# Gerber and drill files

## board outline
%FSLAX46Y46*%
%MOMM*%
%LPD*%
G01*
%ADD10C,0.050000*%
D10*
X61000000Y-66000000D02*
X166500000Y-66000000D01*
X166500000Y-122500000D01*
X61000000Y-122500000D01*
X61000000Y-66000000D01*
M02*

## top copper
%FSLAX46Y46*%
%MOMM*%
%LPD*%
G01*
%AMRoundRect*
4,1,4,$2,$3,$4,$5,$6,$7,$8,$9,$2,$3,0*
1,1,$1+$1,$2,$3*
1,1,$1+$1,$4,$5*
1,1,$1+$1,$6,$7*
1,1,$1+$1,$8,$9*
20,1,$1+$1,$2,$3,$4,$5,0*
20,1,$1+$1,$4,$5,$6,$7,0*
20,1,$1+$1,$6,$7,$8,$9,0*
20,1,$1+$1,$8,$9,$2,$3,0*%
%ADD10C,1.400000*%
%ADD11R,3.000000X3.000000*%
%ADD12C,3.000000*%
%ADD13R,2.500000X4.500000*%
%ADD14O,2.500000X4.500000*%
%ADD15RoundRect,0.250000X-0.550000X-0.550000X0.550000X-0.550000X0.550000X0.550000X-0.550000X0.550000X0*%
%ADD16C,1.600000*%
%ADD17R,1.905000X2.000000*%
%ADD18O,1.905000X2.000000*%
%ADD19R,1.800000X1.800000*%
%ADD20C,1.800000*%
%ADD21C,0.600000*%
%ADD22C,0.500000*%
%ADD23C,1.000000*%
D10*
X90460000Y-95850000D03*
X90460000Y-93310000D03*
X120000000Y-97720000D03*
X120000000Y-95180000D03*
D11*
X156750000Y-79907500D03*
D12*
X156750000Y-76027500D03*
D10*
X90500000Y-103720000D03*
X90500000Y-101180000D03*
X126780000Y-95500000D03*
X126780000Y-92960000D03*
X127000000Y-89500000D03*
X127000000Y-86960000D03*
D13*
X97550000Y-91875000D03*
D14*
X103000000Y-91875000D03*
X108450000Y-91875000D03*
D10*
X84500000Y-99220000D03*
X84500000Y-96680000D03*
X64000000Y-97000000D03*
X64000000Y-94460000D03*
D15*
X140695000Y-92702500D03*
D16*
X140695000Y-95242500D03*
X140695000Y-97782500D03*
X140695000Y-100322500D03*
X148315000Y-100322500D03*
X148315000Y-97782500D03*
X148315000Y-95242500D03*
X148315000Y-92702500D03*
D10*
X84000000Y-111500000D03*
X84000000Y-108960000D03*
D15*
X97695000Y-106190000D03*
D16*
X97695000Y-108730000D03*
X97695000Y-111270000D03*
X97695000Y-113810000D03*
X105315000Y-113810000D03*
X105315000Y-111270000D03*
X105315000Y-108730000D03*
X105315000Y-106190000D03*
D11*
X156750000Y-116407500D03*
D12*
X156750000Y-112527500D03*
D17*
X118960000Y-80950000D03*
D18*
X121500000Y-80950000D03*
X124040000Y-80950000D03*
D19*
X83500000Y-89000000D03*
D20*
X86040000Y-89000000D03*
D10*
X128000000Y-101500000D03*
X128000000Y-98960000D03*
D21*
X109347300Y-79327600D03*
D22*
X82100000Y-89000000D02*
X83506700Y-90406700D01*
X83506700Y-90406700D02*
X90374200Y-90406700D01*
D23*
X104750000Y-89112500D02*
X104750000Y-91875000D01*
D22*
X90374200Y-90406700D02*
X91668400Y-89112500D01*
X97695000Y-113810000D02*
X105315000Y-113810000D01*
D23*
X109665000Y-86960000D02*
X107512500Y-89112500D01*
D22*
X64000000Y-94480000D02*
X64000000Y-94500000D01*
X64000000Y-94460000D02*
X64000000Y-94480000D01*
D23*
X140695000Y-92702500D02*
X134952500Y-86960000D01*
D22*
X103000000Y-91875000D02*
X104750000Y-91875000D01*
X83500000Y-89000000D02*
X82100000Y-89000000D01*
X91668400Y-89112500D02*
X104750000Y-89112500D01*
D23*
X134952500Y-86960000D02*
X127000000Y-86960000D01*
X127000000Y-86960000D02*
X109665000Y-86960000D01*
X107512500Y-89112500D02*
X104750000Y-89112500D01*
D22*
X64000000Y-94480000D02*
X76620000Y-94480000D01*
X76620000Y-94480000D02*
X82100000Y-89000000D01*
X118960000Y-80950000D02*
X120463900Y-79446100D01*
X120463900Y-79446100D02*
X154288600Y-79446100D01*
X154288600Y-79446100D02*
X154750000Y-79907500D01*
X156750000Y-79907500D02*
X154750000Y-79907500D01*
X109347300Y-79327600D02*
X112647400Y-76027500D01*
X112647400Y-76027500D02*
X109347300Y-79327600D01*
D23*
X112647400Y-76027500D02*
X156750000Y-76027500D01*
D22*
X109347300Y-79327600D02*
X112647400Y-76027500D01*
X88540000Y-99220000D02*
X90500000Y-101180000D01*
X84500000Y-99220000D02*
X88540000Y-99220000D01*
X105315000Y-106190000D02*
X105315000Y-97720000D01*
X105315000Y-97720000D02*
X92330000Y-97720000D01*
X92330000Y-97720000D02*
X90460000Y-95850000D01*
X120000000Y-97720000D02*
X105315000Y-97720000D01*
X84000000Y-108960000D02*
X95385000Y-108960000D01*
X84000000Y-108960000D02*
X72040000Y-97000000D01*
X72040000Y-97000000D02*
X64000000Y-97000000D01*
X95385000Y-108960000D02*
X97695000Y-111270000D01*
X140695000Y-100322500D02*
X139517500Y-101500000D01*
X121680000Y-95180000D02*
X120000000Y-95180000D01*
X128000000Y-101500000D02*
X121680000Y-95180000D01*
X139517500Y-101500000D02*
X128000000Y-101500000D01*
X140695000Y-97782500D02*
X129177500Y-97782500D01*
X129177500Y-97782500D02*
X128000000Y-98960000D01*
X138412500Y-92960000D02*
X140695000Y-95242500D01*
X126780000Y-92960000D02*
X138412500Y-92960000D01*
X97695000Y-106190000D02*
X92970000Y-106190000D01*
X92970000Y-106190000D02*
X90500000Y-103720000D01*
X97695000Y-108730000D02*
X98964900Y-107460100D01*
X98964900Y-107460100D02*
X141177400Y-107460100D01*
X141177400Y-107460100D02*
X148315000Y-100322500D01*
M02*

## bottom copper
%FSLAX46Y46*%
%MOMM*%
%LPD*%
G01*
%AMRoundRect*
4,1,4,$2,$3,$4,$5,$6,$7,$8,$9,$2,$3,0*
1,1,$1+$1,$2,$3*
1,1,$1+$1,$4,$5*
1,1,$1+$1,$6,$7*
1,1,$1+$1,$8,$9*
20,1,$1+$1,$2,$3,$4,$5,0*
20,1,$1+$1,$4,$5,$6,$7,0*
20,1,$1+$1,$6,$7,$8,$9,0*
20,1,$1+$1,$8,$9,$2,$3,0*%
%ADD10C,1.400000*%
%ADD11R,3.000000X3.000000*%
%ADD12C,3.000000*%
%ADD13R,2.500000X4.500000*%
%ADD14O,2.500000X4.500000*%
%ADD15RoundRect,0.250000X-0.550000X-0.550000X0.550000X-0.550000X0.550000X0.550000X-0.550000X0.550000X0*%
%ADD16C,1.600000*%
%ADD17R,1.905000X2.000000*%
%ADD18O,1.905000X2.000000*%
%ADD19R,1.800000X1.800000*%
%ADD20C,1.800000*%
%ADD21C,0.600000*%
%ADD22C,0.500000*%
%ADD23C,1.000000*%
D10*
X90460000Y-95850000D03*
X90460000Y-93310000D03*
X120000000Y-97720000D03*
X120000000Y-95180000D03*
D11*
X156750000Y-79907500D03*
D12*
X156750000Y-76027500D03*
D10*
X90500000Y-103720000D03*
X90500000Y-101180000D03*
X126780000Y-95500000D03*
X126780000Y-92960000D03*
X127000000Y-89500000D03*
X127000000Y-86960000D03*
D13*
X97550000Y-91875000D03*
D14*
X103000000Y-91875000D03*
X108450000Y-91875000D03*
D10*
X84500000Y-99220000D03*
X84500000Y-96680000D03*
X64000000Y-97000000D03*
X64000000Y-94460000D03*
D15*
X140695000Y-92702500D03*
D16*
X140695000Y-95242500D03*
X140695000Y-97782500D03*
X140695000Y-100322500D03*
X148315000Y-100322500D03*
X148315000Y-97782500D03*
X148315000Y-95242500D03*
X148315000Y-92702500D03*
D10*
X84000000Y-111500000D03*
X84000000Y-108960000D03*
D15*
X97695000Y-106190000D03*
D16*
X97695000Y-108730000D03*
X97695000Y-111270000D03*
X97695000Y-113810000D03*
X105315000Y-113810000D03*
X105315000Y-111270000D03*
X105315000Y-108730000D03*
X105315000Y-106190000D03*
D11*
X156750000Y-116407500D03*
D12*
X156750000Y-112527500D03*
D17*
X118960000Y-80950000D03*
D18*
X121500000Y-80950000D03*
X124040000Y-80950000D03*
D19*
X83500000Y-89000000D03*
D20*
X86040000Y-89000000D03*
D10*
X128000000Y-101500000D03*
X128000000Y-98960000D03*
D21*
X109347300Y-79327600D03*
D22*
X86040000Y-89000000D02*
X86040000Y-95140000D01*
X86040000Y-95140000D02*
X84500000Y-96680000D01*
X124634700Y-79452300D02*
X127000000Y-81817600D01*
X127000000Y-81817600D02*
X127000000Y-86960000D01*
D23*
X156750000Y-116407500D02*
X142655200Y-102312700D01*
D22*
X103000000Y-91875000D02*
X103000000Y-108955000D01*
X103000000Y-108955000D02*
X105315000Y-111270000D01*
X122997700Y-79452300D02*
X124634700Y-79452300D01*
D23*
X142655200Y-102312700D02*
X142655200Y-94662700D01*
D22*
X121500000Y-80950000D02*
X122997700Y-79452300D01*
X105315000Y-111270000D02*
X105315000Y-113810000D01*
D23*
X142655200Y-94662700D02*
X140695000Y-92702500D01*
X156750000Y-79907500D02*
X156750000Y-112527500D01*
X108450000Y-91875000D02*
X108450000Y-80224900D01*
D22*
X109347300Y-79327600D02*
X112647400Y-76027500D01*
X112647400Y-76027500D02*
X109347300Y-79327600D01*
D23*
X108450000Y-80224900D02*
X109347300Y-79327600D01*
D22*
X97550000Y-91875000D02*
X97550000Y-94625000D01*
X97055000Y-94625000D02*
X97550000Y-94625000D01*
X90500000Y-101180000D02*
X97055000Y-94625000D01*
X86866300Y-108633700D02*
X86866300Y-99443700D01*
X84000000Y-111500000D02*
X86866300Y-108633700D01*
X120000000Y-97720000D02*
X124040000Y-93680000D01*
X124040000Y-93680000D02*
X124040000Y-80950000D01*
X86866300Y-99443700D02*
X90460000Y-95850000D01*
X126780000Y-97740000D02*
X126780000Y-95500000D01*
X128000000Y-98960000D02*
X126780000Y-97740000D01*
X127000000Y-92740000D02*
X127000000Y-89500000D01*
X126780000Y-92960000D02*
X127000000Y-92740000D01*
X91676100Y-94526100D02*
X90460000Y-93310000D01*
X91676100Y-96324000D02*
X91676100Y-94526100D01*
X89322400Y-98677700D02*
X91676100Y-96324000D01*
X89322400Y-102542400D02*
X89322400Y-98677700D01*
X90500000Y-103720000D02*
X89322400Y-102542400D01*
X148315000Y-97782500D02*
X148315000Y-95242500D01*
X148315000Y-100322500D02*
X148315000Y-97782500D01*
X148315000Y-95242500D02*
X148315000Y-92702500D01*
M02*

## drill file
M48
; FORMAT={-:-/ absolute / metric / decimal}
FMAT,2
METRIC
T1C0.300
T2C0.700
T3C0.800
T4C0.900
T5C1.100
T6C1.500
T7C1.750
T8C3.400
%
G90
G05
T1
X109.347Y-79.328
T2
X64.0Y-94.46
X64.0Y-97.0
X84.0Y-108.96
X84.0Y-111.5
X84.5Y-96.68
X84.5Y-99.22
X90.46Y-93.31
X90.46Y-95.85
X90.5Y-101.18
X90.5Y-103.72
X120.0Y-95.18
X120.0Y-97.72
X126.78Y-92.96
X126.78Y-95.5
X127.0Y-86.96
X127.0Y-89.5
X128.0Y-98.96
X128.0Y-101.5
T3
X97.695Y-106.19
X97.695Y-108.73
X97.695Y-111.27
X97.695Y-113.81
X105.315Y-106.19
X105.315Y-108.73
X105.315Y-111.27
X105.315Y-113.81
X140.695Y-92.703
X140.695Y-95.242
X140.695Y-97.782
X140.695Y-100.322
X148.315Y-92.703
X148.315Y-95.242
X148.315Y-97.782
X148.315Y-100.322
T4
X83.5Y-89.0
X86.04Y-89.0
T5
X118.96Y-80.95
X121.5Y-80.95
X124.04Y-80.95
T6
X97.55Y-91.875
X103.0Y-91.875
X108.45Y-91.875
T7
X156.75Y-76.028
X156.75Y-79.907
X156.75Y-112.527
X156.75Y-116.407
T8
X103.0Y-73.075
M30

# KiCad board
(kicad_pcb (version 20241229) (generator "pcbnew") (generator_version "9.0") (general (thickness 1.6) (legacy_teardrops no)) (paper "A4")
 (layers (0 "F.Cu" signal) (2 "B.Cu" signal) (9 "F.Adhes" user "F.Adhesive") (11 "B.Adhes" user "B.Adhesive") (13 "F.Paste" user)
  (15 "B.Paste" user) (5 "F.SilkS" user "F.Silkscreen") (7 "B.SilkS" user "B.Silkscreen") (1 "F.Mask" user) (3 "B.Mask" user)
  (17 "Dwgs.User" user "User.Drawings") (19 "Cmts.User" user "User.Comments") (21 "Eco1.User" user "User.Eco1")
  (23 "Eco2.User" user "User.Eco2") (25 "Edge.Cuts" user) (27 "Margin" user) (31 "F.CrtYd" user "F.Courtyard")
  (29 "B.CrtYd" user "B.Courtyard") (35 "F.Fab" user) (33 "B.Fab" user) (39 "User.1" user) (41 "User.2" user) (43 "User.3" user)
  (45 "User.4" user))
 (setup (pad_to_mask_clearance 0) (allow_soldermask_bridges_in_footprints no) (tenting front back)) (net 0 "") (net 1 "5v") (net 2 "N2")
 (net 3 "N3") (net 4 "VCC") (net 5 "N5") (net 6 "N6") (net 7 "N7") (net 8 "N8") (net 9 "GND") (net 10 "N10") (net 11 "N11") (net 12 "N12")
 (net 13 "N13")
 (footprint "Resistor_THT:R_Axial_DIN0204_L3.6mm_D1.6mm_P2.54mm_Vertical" (layer "F.Cu") (at 90.46 95.85 90)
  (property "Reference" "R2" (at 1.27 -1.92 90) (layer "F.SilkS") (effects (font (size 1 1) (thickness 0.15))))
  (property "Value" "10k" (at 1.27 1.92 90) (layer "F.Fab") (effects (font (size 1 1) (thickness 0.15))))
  (pad "1" thru_hole circle (at 0 0 90) (size 1.4 1.4) (drill 0.7) (layers "*.Cu" "*.Mask") (remove_unused_layers no) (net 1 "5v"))
  (pad "2" thru_hole circle (at 2.54 0 90) (size 1.4 1.4) (drill 0.7) (layers "*.Cu" "*.Mask") (remove_unused_layers no) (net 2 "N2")))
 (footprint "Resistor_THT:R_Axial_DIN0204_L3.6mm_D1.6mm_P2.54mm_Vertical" (layer "F.Cu") (at 120 97.72 90)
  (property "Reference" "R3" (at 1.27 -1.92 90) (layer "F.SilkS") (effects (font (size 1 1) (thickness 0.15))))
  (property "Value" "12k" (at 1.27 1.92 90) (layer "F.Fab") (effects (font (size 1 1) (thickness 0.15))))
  (pad "1" thru_hole circle (at 0 0 90) (size 1.4 1.4) (drill 0.7) (layers "*.Cu" "*.Mask") (remove_unused_layers no) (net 1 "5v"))
  (pad "2" thru_hole circle (at 2.54 0 90) (size 1.4 1.4) (drill 0.7) (layers "*.Cu" "*.Mask") (remove_unused_layers no) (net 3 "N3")))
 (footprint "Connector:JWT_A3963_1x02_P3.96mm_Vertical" (layer "F.Cu") (at 156.75 79.9075 90)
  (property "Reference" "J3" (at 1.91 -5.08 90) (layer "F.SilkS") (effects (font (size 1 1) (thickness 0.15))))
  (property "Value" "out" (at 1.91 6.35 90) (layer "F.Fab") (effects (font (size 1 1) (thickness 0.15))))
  (pad "1" thru_hole rect (at 0 0 90) (size 3 3) (drill 1.75) (layers "*.Cu" "*.Mask") (remove_unused_layers no) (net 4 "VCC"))
  (pad "2" thru_hole circle (at 3.88 0 90) (size 3 3) (drill 1.75) (layers "*.Cu" "*.Mask") (remove_unused_layers no) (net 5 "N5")))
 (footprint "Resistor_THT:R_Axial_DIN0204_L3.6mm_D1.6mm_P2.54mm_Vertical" (layer "F.Cu") (at 90.5 103.72 90)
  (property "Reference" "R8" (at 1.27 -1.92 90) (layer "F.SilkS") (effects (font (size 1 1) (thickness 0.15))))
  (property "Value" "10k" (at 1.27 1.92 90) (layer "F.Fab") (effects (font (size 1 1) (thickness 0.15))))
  (pad "1" thru_hole circle (at 0 0 90) (size 1.4 1.4) (drill 0.7) (layers "*.Cu" "*.Mask") (remove_unused_layers no) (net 2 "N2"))
  (pad "2" thru_hole circle (at 2.54 0 90) (size 1.4 1.4) (drill 0.7) (layers "*.Cu" "*.Mask") (remove_unused_layers no) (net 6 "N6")))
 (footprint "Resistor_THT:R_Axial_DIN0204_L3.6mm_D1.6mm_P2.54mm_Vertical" (layer "F.Cu") (at 126.78 95.5 90)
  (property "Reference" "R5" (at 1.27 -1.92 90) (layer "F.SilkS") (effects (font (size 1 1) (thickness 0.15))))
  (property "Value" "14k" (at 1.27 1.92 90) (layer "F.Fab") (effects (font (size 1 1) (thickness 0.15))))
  (pad "1" thru_hole circle (at 0 0 90) (size 1.4 1.4) (drill 0.7) (layers "*.Cu" "*.Mask") (remove_unused_layers no) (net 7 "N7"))
  (pad "2" thru_hole circle (at 2.54 0 90) (size 1.4 1.4) (drill 0.7) (layers "*.Cu" "*.Mask") (remove_unused_layers no) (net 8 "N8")))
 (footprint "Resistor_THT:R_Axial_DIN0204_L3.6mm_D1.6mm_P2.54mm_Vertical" (layer "F.Cu") (at 127 89.5 90)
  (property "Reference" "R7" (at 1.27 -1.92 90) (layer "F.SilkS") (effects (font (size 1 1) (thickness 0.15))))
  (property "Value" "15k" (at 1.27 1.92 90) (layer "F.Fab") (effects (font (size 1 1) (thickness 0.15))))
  (pad "1" thru_hole circle (at 0 0 90) (size 1.4 1.4) (drill 0.7) (layers "*.Cu" "*.Mask") (remove_unused_layers no) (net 8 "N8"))
  (pad "2" thru_hole circle (at 2.54 0 90) (size 1.4 1.4) (drill 0.7) (layers "*.Cu" "*.Mask") (remove_unused_layers no) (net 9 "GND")))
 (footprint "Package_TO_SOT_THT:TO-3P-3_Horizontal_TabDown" (layer "F.Cu") (at 97.55 91.875)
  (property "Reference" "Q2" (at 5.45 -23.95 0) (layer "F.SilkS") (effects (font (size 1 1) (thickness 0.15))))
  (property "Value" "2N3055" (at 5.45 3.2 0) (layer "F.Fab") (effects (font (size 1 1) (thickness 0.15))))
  (pad "" np_thru_hole circle (at 5.45 -18.8) (size 3.4 3.4) (drill 3.4) (layers "*.Cu" "*.Mask"))
  (pad "1" thru_hole rect (at 0 0) (size 2.5 4.5) (drill 1.5) (layers "*.Cu" "*.Mask") (remove_unused_layers no) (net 6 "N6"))
  (pad "2" thru_hole oval (at 5.45 0) (size 2.5 4.5) (drill 1.5) (layers "*.Cu" "*.Mask") (remove_unused_layers no) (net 9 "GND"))
  (pad "3" thru_hole oval (at 10.9 0) (size 2.5 4.5) (drill 1.5) (layers "*.Cu" "*.Mask") (remove_unused_layers no) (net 5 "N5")))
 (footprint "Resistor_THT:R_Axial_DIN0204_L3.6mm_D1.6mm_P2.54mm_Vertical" (layer "F.Cu") (at 84.5 99.22 90)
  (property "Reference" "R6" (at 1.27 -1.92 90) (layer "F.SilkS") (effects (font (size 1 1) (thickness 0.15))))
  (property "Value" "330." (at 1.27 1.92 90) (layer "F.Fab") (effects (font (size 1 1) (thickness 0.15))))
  (pad "1" thru_hole circle (at 0 0 90) (size 1.4 1.4) (drill 0.7) (layers "*.Cu" "*.Mask") (remove_unused_layers no) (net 6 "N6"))
  (pad "2" thru_hole circle (at 2.54 0 90) (size 1.4 1.4) (drill 0.7) (layers "*.Cu" "*.Mask") (remove_unused_layers no) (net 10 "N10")))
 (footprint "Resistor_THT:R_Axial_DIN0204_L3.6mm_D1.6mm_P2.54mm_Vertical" (layer "F.Cu") (at 64 97 90)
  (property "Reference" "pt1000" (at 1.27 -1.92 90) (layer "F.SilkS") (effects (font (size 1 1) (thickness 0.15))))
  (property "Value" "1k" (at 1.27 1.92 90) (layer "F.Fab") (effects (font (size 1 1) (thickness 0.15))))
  (pad "1" thru_hole circle (at 0 0 90) (size 1.4 1.4) (drill 0.7) (layers "*.Cu" "*.Mask") (remove_unused_layers no) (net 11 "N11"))
  (pad "2" thru_hole circle (at 2.54 0 90) (size 1.4 1.4) (drill 0.7) (layers "*.Cu" "*.Mask") (remove_unused_layers no) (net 9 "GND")))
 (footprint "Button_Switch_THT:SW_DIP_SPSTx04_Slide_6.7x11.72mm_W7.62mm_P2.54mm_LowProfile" (layer "F.Cu") (at 140.695 92.7025)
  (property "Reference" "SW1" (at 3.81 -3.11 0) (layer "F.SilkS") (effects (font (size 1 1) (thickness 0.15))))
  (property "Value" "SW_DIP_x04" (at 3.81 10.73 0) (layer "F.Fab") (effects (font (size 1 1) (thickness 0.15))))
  (pad "1" thru_hole roundrect (at 0 0) (size 1.6 1.6) (drill 0.8) (layers "*.Cu" "*.Mask") (remove_unused_layers no)
   (roundrect_rratio 0.15625) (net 9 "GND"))
  (pad "2" thru_hole circle (at 0 2.54) (size 1.6 1.6) (drill 0.8) (layers "*.Cu" "*.Mask") (remove_unused_layers no) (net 8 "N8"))
  (pad "3" thru_hole circle (at 0 5.08) (size 1.6 1.6) (drill 0.8) (layers "*.Cu" "*.Mask") (remove_unused_layers no) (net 7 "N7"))
  (pad "4" thru_hole circle (at 0 7.62) (size 1.6 1.6) (drill 0.8) (layers "*.Cu" "*.Mask") (remove_unused_layers no) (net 3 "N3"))
  (pad "5" thru_hole circle (at 7.62 7.62) (size 1.6 1.6) (drill 0.8) (layers "*.Cu" "*.Mask") (remove_unused_layers no) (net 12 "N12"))
  (pad "6" thru_hole circle (at 7.62 5.08) (size 1.6 1.6) (drill 0.8) (layers "*.Cu" "*.Mask") (remove_unused_layers no) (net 12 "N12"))
  (pad "7" thru_hole circle (at 7.62 2.54) (size 1.6 1.6) (drill 0.8) (layers "*.Cu" "*.Mask") (remove_unused_layers no) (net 12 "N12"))
  (pad "8" thru_hole circle (at 7.62 0) (size 1.6 1.6) (drill 0.8) (layers "*.Cu" "*.Mask") (remove_unused_layers no) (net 12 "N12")))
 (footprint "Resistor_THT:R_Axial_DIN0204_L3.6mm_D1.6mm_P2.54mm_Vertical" (layer "F.Cu") (at 84 111.5 90)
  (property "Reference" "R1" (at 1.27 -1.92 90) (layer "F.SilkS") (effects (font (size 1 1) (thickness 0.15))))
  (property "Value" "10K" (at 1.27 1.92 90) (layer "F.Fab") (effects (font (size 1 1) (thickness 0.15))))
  (pad "1" thru_hole circle (at 0 0 90) (size 1.4 1.4) (drill 0.7) (layers "*.Cu" "*.Mask") (remove_unused_layers no) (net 1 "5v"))
  (pad "2" thru_hole circle (at 2.54 0 90) (size 1.4 1.4) (drill 0.7) (layers "*.Cu" "*.Mask") (remove_unused_layers no) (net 11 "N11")))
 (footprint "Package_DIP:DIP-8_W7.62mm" (layer "F.Cu") (at 97.695 106.19)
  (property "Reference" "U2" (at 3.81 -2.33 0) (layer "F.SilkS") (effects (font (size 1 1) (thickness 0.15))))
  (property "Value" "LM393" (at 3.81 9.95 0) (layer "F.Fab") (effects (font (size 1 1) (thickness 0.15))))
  (pad "1" thru_hole roundrect (at 0 0) (size 1.6 1.6) (drill 0.8) (layers "*.Cu" "*.Mask") (remove_unused_layers no)
   (roundrect_rratio 0.15625) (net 2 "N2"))
  (pad "2" thru_hole circle (at 0 2.54) (size 1.6 1.6) (drill 0.8) (layers "*.Cu" "*.Mask") (remove_unused_layers no) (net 12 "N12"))
  (pad "3" thru_hole circle (at 0 5.08) (size 1.6 1.6) (drill 0.8) (layers "*.Cu" "*.Mask") (remove_unused_layers no) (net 11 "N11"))
  (pad "4" thru_hole circle (at 0 7.62) (size 1.6 1.6) (drill 0.8) (layers "*.Cu" "*.Mask") (remove_unused_layers no) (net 9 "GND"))
  (pad "5" thru_hole circle (at 7.62 7.62) (size 1.6 1.6) (drill 0.8) (layers "*.Cu" "*.Mask") (remove_unused_layers no) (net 9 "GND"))
  (pad "6" thru_hole circle (at 7.62 5.08) (size 1.6 1.6) (drill 0.8) (layers "*.Cu" "*.Mask") (remove_unused_layers no) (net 9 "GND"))
  (pad "7" thru_hole circle (at 7.62 2.54) (size 1.6 1.6) (drill 0.8) (layers "*.Cu" "*.Mask") (remove_unused_layers no) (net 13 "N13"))
  (pad "8" thru_hole circle (at 7.62 0) (size 1.6 1.6) (drill 0.8) (layers "*.Cu" "*.Mask") (remove_unused_layers no) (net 1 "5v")))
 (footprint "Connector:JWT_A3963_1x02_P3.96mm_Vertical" (layer "F.Cu") (at 156.75 116.4075 90)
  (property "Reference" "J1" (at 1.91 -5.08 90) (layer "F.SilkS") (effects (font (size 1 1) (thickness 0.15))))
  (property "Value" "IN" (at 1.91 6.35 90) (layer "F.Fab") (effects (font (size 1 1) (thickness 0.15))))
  (pad "1" thru_hole rect (at 0 0 90) (size 3 3) (drill 1.75) (layers "*.Cu" "*.Mask") (remove_unused_layers no) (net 9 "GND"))
  (pad "2" thru_hole circle (at 3.88 0 90) (size 3 3) (drill 1.75) (layers "*.Cu" "*.Mask") (remove_unused_layers no) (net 4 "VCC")))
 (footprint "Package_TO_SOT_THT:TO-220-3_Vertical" (layer "F.Cu") (at 118.96 80.95)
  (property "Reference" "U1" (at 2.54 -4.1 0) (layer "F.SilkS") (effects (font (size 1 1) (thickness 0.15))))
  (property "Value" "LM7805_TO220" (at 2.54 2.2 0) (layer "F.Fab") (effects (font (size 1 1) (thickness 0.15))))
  (pad "1" thru_hole rect (at 0 0) (size 1.905 2) (drill 1.1) (layers "*.Cu" "*.Mask") (remove_unused_layers no) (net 4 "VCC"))
  (pad "2" thru_hole oval (at 2.54 0) (size 1.905 2) (drill 1.1) (layers "*.Cu" "*.Mask") (remove_unused_layers no) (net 9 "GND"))
  (pad "3" thru_hole oval (at 5.08 0) (size 1.905 2) (drill 1.1) (layers "*.Cu" "*.Mask") (remove_unused_layers no) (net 1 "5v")))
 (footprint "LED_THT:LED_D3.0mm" (layer "F.Cu") (at 83.5 89)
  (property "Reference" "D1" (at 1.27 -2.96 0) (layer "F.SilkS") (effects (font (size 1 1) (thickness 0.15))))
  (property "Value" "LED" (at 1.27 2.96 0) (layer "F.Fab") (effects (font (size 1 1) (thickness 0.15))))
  (pad "1" thru_hole rect (at 0 0) (size 1.8 1.8) (drill 0.9) (layers "*.Cu" "*.Mask") (remove_unused_layers no) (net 9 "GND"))
  (pad "2" thru_hole circle (at 2.54 0) (size 1.8 1.8) (drill 0.9) (layers "*.Cu" "*.Mask") (remove_unused_layers no) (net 10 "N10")))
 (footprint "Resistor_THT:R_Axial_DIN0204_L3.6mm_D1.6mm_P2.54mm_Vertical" (layer "F.Cu") (at 128 101.5 90)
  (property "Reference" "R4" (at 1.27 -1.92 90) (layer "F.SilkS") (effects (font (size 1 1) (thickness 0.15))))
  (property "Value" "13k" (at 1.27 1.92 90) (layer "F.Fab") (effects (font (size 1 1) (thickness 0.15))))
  (pad "1" thru_hole circle (at 0 0 90) (size 1.4 1.4) (drill 0.7) (layers "*.Cu" "*.Mask") (remove_unused_layers no) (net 3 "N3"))
  (pad "2" thru_hole circle (at 2.54 0 90) (size 1.4 1.4) (drill 0.7) (layers "*.Cu" "*.Mask") (remove_unused_layers no) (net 7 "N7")))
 (gr_rect (start 61 66) (end 166.5 122.5) (stroke (width 0.05) (type default)) (fill no) (layer "Edge.Cuts"))
 (segment (start 86.04 89) (end 86.04 95.14) (width 0.5) (layer "B.Cu") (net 10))
 (segment (start 86.04 95.14) (end 84.5 96.68) (width 0.5) (layer "B.Cu") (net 10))
 (segment (start 82.1 89) (end 83.5067 90.4067) (width 0.5) (layer "F.Cu") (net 9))
 (segment (start 83.5067 90.4067) (end 90.3742 90.4067) (width 0.5) (layer "F.Cu") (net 9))
 (segment (start 104.75 89.1125) (end 104.75 91.875) (width 1) (layer "F.Cu") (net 9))
 (segment (start 90.3742 90.4067) (end 91.6684 89.1125) (width 0.5) (layer "F.Cu") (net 9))
 (segment (start 97.695 113.81) (end 105.315 113.81) (width 0.5) (layer "F.Cu") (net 9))
 (segment (start 109.665 86.96) (end 107.5125 89.1125) (width 1) (layer "F.Cu") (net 9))
 (segment (start 64 94.48) (end 64 94.5) (width 0.5) (layer "F.Cu") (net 9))
 (segment (start 64 94.46) (end 64 94.48) (width 0.5) (layer "F.Cu") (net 9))
 (segment (start 140.695 92.7025) (end 134.9525 86.96) (width 1) (layer "F.Cu") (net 9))
 (segment (start 103 91.875) (end 104.75 91.875) (width 0.5) (layer "F.Cu") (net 9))
 (segment (start 83.5 89) (end 82.1 89) (width 0.5) (layer "F.Cu") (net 9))
 (segment (start 91.6684 89.1125) (end 104.75 89.1125) (width 0.5) (layer "F.Cu") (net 9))
 (segment (start 134.9525 86.96) (end 127 86.96) (width 1) (layer "F.Cu") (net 9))
 (segment (start 127 86.96) (end 109.665 86.96) (width 1) (layer "F.Cu") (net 9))
 (segment (start 107.5125 89.1125) (end 104.75 89.1125) (width 1) (layer "F.Cu") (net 9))
 (segment (start 64 94.48) (end 76.62 94.48) (width 0.5) (layer "F.Cu") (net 9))
 (segment (start 76.62 94.48) (end 82.1 89) (width 0.5) (layer "F.Cu") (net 9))
 (segment (start 124.6347 79.4523) (end 127 81.8176) (width 0.5) (layer "B.Cu") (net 9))
 (segment (start 127 81.8176) (end 127 86.96) (width 0.5) (layer "B.Cu") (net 9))
 (segment (start 156.75 116.4075) (end 142.6552 102.3127) (width 1) (layer "B.Cu") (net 9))
 (segment (start 103 91.875) (end 103 108.955) (width 0.5) (layer "B.Cu") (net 9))
 (segment (start 103 108.955) (end 105.315 111.27) (width 0.5) (layer "B.Cu") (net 9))
 (segment (start 122.9977 79.4523) (end 124.6347 79.4523) (width 0.5) (layer "B.Cu") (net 9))
 (segment (start 142.6552 102.3127) (end 142.6552 94.6627) (width 1) (layer "B.Cu") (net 9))
 (segment (start 121.5 80.95) (end 122.9977 79.4523) (width 0.5) (layer "B.Cu") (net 9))
 (segment (start 105.315 111.27) (end 105.315 113.81) (width 0.5) (layer "B.Cu") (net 9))
 (segment (start 142.6552 94.6627) (end 140.695 92.7025) (width 1) (layer "B.Cu") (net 9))
 (segment (start 118.96 80.95) (end 120.4639 79.4461) (width 0.5) (layer "F.Cu") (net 4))
 (segment (start 120.4639 79.4461) (end 154.2886 79.4461) (width 0.5) (layer "F.Cu") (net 4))
 (segment (start 154.2886 79.4461) (end 154.75 79.9075) (width 0.5) (layer "F.Cu") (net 4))
 (segment (start 156.75 79.9075) (end 154.75 79.9075) (width 0.5) (layer "F.Cu") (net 4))
 (segment (start 156.75 79.9075) (end 156.75 112.5275) (width 1) (layer "B.Cu") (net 4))
 (segment (start 109.3473 79.3276) (end 112.6474 76.0275) (width 0.5) (layer "F.Cu") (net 5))
 (segment (start 112.6474 76.0275) (end 109.3473 79.3276) (width 0.5) (layer "F.Cu") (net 5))
 (segment (start 112.6474 76.0275) (end 156.75 76.0275) (width 1) (layer "F.Cu") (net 5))
 (segment (start 109.3473 79.3276) (end 112.6474 76.0275) (width 0.5) (layer "F.Cu") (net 5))
 (via (at 109.3473 79.3276) (size 0.6) (drill 0.3) (layers "F.Cu" "B.Cu") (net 5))
 (segment (start 108.45 91.875) (end 108.45 80.2249) (width 1) (layer "B.Cu") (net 5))
 (segment (start 109.3473 79.3276) (end 112.6474 76.0275) (width 0.5) (layer "B.Cu") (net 5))
 (segment (start 112.6474 76.0275) (end 109.3473 79.3276) (width 0.5) (layer "B.Cu") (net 5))
 (segment (start 108.45 80.2249) (end 109.3473 79.3276) (width 1) (layer "B.Cu") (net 5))
 (segment (start 88.54 99.22) (end 90.5 101.18) (width 0.5) (layer "F.Cu") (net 6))
 (segment (start 84.5 99.22) (end 88.54 99.22) (width 0.5) (layer "F.Cu") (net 6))
 (segment (start 97.55 91.875) (end 97.55 94.625) (width 0.5) (layer "B.Cu") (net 6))
 (segment (start 97.055 94.625) (end 97.55 94.625) (width 0.5) (layer "B.Cu") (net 6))
 (segment (start 90.5 101.18) (end 97.055 94.625) (width 0.5) (layer "B.Cu") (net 6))
 (segment (start 105.315 106.19) (end 105.315 97.72) (width 0.5) (layer "F.Cu") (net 1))
 (segment (start 105.315 97.72) (end 92.33 97.72) (width 0.5) (layer "F.Cu") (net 1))
 (segment (start 92.33 97.72) (end 90.46 95.85) (width 0.5) (layer "F.Cu") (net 1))
 (segment (start 120 97.72) (end 105.315 97.72) (width 0.5) (layer "F.Cu") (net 1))
 (segment (start 86.8663 108.6337) (end 86.8663 99.4437) (width 0.5) (layer "B.Cu") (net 1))
 (segment (start 84 111.5) (end 86.8663 108.6337) (width 0.5) (layer "B.Cu") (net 1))
 (segment (start 120 97.72) (end 124.04 93.68) (width 0.5) (layer "B.Cu") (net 1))
 (segment (start 124.04 93.68) (end 124.04 80.95) (width 0.5) (layer "B.Cu") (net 1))
 (segment (start 86.8663 99.4437) (end 90.46 95.85) (width 0.5) (layer "B.Cu") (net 1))
 (segment (start 84 108.96) (end 95.385 108.96) (width 0.5) (layer "F.Cu") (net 11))
 (segment (start 84 108.96) (end 72.04 97) (width 0.5) (layer "F.Cu") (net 11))
 (segment (start 72.04 97) (end 64 97) (width 0.5) (layer "F.Cu") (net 11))
 (segment (start 95.385 108.96) (end 97.695 111.27) (width 0.5) (layer "F.Cu") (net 11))
 (segment (start 140.695 100.3225) (end 139.5175 101.5) (width 0.5) (layer "F.Cu") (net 3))
 (segment (start 121.68 95.18) (end 120 95.18) (width 0.5) (layer "F.Cu") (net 3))
 (segment (start 128 101.5) (end 121.68 95.18) (width 0.5) (layer "F.Cu") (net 3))
 (segment (start 139.5175 101.5) (end 128 101.5) (width 0.5) (layer "F.Cu") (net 3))
 (segment (start 140.695 97.7825) (end 129.1775 97.7825) (width 0.5) (layer "F.Cu") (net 7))
 (segment (start 129.1775 97.7825) (end 128 98.96) (width 0.5) (layer "F.Cu") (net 7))
 (segment (start 126.78 97.74) (end 126.78 95.5) (width 0.5) (layer "B.Cu") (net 7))
 (segment (start 128 98.96) (end 126.78 97.74) (width 0.5) (layer "B.Cu") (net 7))
 (segment (start 138.4125 92.96) (end 140.695 95.2425) (width 0.5) (layer "F.Cu") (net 8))
 (segment (start 126.78 92.96) (end 138.4125 92.96) (width 0.5) (layer "F.Cu") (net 8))
 (segment (start 127 92.74) (end 127 89.5) (width 0.5) (layer "B.Cu") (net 8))
 (segment (start 126.78 92.96) (end 127 92.74) (width 0.5) (layer "B.Cu") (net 8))
 (segment (start 97.695 106.19) (end 92.97 106.19) (width 0.5) (layer "F.Cu") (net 2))
 (segment (start 92.97 106.19) (end 90.5 103.72) (width 0.5) (layer "F.Cu") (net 2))
 (segment (start 91.6761 94.5261) (end 90.46 93.31) (width 0.5) (layer "B.Cu") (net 2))
 (segment (start 91.6761 96.324) (end 91.6761 94.5261) (width 0.5) (layer "B.Cu") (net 2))
 (segment (start 89.3224 98.6777) (end 91.6761 96.324) (width 0.5) (layer "B.Cu") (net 2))
 (segment (start 89.3224 102.5424) (end 89.3224 98.6777) (width 0.5) (layer "B.Cu") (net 2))
 (segment (start 90.5 103.72) (end 89.3224 102.5424) (width 0.5) (layer "B.Cu") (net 2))
 (segment (start 97.695 108.73) (end 98.9649 107.4601) (width 0.5) (layer "F.Cu") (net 12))
 (segment (start 98.9649 107.4601) (end 141.1774 107.4601) (width 0.5) (layer "F.Cu") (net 12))
 (segment (start 141.1774 107.4601) (end 148.315 100.3225) (width 0.5) (layer "F.Cu") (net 12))
 (segment (start 148.315 97.7825) (end 148.315 95.2425) (width 0.5) (layer "B.Cu") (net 12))
 (segment (start 148.315 100.3225) (end 148.315 97.7825) (width 0.5) (layer "B.Cu") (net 12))
 (segment (start 148.315 95.2425) (end 148.315 92.7025) (width 0.5) (layer "B.Cu") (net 12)))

